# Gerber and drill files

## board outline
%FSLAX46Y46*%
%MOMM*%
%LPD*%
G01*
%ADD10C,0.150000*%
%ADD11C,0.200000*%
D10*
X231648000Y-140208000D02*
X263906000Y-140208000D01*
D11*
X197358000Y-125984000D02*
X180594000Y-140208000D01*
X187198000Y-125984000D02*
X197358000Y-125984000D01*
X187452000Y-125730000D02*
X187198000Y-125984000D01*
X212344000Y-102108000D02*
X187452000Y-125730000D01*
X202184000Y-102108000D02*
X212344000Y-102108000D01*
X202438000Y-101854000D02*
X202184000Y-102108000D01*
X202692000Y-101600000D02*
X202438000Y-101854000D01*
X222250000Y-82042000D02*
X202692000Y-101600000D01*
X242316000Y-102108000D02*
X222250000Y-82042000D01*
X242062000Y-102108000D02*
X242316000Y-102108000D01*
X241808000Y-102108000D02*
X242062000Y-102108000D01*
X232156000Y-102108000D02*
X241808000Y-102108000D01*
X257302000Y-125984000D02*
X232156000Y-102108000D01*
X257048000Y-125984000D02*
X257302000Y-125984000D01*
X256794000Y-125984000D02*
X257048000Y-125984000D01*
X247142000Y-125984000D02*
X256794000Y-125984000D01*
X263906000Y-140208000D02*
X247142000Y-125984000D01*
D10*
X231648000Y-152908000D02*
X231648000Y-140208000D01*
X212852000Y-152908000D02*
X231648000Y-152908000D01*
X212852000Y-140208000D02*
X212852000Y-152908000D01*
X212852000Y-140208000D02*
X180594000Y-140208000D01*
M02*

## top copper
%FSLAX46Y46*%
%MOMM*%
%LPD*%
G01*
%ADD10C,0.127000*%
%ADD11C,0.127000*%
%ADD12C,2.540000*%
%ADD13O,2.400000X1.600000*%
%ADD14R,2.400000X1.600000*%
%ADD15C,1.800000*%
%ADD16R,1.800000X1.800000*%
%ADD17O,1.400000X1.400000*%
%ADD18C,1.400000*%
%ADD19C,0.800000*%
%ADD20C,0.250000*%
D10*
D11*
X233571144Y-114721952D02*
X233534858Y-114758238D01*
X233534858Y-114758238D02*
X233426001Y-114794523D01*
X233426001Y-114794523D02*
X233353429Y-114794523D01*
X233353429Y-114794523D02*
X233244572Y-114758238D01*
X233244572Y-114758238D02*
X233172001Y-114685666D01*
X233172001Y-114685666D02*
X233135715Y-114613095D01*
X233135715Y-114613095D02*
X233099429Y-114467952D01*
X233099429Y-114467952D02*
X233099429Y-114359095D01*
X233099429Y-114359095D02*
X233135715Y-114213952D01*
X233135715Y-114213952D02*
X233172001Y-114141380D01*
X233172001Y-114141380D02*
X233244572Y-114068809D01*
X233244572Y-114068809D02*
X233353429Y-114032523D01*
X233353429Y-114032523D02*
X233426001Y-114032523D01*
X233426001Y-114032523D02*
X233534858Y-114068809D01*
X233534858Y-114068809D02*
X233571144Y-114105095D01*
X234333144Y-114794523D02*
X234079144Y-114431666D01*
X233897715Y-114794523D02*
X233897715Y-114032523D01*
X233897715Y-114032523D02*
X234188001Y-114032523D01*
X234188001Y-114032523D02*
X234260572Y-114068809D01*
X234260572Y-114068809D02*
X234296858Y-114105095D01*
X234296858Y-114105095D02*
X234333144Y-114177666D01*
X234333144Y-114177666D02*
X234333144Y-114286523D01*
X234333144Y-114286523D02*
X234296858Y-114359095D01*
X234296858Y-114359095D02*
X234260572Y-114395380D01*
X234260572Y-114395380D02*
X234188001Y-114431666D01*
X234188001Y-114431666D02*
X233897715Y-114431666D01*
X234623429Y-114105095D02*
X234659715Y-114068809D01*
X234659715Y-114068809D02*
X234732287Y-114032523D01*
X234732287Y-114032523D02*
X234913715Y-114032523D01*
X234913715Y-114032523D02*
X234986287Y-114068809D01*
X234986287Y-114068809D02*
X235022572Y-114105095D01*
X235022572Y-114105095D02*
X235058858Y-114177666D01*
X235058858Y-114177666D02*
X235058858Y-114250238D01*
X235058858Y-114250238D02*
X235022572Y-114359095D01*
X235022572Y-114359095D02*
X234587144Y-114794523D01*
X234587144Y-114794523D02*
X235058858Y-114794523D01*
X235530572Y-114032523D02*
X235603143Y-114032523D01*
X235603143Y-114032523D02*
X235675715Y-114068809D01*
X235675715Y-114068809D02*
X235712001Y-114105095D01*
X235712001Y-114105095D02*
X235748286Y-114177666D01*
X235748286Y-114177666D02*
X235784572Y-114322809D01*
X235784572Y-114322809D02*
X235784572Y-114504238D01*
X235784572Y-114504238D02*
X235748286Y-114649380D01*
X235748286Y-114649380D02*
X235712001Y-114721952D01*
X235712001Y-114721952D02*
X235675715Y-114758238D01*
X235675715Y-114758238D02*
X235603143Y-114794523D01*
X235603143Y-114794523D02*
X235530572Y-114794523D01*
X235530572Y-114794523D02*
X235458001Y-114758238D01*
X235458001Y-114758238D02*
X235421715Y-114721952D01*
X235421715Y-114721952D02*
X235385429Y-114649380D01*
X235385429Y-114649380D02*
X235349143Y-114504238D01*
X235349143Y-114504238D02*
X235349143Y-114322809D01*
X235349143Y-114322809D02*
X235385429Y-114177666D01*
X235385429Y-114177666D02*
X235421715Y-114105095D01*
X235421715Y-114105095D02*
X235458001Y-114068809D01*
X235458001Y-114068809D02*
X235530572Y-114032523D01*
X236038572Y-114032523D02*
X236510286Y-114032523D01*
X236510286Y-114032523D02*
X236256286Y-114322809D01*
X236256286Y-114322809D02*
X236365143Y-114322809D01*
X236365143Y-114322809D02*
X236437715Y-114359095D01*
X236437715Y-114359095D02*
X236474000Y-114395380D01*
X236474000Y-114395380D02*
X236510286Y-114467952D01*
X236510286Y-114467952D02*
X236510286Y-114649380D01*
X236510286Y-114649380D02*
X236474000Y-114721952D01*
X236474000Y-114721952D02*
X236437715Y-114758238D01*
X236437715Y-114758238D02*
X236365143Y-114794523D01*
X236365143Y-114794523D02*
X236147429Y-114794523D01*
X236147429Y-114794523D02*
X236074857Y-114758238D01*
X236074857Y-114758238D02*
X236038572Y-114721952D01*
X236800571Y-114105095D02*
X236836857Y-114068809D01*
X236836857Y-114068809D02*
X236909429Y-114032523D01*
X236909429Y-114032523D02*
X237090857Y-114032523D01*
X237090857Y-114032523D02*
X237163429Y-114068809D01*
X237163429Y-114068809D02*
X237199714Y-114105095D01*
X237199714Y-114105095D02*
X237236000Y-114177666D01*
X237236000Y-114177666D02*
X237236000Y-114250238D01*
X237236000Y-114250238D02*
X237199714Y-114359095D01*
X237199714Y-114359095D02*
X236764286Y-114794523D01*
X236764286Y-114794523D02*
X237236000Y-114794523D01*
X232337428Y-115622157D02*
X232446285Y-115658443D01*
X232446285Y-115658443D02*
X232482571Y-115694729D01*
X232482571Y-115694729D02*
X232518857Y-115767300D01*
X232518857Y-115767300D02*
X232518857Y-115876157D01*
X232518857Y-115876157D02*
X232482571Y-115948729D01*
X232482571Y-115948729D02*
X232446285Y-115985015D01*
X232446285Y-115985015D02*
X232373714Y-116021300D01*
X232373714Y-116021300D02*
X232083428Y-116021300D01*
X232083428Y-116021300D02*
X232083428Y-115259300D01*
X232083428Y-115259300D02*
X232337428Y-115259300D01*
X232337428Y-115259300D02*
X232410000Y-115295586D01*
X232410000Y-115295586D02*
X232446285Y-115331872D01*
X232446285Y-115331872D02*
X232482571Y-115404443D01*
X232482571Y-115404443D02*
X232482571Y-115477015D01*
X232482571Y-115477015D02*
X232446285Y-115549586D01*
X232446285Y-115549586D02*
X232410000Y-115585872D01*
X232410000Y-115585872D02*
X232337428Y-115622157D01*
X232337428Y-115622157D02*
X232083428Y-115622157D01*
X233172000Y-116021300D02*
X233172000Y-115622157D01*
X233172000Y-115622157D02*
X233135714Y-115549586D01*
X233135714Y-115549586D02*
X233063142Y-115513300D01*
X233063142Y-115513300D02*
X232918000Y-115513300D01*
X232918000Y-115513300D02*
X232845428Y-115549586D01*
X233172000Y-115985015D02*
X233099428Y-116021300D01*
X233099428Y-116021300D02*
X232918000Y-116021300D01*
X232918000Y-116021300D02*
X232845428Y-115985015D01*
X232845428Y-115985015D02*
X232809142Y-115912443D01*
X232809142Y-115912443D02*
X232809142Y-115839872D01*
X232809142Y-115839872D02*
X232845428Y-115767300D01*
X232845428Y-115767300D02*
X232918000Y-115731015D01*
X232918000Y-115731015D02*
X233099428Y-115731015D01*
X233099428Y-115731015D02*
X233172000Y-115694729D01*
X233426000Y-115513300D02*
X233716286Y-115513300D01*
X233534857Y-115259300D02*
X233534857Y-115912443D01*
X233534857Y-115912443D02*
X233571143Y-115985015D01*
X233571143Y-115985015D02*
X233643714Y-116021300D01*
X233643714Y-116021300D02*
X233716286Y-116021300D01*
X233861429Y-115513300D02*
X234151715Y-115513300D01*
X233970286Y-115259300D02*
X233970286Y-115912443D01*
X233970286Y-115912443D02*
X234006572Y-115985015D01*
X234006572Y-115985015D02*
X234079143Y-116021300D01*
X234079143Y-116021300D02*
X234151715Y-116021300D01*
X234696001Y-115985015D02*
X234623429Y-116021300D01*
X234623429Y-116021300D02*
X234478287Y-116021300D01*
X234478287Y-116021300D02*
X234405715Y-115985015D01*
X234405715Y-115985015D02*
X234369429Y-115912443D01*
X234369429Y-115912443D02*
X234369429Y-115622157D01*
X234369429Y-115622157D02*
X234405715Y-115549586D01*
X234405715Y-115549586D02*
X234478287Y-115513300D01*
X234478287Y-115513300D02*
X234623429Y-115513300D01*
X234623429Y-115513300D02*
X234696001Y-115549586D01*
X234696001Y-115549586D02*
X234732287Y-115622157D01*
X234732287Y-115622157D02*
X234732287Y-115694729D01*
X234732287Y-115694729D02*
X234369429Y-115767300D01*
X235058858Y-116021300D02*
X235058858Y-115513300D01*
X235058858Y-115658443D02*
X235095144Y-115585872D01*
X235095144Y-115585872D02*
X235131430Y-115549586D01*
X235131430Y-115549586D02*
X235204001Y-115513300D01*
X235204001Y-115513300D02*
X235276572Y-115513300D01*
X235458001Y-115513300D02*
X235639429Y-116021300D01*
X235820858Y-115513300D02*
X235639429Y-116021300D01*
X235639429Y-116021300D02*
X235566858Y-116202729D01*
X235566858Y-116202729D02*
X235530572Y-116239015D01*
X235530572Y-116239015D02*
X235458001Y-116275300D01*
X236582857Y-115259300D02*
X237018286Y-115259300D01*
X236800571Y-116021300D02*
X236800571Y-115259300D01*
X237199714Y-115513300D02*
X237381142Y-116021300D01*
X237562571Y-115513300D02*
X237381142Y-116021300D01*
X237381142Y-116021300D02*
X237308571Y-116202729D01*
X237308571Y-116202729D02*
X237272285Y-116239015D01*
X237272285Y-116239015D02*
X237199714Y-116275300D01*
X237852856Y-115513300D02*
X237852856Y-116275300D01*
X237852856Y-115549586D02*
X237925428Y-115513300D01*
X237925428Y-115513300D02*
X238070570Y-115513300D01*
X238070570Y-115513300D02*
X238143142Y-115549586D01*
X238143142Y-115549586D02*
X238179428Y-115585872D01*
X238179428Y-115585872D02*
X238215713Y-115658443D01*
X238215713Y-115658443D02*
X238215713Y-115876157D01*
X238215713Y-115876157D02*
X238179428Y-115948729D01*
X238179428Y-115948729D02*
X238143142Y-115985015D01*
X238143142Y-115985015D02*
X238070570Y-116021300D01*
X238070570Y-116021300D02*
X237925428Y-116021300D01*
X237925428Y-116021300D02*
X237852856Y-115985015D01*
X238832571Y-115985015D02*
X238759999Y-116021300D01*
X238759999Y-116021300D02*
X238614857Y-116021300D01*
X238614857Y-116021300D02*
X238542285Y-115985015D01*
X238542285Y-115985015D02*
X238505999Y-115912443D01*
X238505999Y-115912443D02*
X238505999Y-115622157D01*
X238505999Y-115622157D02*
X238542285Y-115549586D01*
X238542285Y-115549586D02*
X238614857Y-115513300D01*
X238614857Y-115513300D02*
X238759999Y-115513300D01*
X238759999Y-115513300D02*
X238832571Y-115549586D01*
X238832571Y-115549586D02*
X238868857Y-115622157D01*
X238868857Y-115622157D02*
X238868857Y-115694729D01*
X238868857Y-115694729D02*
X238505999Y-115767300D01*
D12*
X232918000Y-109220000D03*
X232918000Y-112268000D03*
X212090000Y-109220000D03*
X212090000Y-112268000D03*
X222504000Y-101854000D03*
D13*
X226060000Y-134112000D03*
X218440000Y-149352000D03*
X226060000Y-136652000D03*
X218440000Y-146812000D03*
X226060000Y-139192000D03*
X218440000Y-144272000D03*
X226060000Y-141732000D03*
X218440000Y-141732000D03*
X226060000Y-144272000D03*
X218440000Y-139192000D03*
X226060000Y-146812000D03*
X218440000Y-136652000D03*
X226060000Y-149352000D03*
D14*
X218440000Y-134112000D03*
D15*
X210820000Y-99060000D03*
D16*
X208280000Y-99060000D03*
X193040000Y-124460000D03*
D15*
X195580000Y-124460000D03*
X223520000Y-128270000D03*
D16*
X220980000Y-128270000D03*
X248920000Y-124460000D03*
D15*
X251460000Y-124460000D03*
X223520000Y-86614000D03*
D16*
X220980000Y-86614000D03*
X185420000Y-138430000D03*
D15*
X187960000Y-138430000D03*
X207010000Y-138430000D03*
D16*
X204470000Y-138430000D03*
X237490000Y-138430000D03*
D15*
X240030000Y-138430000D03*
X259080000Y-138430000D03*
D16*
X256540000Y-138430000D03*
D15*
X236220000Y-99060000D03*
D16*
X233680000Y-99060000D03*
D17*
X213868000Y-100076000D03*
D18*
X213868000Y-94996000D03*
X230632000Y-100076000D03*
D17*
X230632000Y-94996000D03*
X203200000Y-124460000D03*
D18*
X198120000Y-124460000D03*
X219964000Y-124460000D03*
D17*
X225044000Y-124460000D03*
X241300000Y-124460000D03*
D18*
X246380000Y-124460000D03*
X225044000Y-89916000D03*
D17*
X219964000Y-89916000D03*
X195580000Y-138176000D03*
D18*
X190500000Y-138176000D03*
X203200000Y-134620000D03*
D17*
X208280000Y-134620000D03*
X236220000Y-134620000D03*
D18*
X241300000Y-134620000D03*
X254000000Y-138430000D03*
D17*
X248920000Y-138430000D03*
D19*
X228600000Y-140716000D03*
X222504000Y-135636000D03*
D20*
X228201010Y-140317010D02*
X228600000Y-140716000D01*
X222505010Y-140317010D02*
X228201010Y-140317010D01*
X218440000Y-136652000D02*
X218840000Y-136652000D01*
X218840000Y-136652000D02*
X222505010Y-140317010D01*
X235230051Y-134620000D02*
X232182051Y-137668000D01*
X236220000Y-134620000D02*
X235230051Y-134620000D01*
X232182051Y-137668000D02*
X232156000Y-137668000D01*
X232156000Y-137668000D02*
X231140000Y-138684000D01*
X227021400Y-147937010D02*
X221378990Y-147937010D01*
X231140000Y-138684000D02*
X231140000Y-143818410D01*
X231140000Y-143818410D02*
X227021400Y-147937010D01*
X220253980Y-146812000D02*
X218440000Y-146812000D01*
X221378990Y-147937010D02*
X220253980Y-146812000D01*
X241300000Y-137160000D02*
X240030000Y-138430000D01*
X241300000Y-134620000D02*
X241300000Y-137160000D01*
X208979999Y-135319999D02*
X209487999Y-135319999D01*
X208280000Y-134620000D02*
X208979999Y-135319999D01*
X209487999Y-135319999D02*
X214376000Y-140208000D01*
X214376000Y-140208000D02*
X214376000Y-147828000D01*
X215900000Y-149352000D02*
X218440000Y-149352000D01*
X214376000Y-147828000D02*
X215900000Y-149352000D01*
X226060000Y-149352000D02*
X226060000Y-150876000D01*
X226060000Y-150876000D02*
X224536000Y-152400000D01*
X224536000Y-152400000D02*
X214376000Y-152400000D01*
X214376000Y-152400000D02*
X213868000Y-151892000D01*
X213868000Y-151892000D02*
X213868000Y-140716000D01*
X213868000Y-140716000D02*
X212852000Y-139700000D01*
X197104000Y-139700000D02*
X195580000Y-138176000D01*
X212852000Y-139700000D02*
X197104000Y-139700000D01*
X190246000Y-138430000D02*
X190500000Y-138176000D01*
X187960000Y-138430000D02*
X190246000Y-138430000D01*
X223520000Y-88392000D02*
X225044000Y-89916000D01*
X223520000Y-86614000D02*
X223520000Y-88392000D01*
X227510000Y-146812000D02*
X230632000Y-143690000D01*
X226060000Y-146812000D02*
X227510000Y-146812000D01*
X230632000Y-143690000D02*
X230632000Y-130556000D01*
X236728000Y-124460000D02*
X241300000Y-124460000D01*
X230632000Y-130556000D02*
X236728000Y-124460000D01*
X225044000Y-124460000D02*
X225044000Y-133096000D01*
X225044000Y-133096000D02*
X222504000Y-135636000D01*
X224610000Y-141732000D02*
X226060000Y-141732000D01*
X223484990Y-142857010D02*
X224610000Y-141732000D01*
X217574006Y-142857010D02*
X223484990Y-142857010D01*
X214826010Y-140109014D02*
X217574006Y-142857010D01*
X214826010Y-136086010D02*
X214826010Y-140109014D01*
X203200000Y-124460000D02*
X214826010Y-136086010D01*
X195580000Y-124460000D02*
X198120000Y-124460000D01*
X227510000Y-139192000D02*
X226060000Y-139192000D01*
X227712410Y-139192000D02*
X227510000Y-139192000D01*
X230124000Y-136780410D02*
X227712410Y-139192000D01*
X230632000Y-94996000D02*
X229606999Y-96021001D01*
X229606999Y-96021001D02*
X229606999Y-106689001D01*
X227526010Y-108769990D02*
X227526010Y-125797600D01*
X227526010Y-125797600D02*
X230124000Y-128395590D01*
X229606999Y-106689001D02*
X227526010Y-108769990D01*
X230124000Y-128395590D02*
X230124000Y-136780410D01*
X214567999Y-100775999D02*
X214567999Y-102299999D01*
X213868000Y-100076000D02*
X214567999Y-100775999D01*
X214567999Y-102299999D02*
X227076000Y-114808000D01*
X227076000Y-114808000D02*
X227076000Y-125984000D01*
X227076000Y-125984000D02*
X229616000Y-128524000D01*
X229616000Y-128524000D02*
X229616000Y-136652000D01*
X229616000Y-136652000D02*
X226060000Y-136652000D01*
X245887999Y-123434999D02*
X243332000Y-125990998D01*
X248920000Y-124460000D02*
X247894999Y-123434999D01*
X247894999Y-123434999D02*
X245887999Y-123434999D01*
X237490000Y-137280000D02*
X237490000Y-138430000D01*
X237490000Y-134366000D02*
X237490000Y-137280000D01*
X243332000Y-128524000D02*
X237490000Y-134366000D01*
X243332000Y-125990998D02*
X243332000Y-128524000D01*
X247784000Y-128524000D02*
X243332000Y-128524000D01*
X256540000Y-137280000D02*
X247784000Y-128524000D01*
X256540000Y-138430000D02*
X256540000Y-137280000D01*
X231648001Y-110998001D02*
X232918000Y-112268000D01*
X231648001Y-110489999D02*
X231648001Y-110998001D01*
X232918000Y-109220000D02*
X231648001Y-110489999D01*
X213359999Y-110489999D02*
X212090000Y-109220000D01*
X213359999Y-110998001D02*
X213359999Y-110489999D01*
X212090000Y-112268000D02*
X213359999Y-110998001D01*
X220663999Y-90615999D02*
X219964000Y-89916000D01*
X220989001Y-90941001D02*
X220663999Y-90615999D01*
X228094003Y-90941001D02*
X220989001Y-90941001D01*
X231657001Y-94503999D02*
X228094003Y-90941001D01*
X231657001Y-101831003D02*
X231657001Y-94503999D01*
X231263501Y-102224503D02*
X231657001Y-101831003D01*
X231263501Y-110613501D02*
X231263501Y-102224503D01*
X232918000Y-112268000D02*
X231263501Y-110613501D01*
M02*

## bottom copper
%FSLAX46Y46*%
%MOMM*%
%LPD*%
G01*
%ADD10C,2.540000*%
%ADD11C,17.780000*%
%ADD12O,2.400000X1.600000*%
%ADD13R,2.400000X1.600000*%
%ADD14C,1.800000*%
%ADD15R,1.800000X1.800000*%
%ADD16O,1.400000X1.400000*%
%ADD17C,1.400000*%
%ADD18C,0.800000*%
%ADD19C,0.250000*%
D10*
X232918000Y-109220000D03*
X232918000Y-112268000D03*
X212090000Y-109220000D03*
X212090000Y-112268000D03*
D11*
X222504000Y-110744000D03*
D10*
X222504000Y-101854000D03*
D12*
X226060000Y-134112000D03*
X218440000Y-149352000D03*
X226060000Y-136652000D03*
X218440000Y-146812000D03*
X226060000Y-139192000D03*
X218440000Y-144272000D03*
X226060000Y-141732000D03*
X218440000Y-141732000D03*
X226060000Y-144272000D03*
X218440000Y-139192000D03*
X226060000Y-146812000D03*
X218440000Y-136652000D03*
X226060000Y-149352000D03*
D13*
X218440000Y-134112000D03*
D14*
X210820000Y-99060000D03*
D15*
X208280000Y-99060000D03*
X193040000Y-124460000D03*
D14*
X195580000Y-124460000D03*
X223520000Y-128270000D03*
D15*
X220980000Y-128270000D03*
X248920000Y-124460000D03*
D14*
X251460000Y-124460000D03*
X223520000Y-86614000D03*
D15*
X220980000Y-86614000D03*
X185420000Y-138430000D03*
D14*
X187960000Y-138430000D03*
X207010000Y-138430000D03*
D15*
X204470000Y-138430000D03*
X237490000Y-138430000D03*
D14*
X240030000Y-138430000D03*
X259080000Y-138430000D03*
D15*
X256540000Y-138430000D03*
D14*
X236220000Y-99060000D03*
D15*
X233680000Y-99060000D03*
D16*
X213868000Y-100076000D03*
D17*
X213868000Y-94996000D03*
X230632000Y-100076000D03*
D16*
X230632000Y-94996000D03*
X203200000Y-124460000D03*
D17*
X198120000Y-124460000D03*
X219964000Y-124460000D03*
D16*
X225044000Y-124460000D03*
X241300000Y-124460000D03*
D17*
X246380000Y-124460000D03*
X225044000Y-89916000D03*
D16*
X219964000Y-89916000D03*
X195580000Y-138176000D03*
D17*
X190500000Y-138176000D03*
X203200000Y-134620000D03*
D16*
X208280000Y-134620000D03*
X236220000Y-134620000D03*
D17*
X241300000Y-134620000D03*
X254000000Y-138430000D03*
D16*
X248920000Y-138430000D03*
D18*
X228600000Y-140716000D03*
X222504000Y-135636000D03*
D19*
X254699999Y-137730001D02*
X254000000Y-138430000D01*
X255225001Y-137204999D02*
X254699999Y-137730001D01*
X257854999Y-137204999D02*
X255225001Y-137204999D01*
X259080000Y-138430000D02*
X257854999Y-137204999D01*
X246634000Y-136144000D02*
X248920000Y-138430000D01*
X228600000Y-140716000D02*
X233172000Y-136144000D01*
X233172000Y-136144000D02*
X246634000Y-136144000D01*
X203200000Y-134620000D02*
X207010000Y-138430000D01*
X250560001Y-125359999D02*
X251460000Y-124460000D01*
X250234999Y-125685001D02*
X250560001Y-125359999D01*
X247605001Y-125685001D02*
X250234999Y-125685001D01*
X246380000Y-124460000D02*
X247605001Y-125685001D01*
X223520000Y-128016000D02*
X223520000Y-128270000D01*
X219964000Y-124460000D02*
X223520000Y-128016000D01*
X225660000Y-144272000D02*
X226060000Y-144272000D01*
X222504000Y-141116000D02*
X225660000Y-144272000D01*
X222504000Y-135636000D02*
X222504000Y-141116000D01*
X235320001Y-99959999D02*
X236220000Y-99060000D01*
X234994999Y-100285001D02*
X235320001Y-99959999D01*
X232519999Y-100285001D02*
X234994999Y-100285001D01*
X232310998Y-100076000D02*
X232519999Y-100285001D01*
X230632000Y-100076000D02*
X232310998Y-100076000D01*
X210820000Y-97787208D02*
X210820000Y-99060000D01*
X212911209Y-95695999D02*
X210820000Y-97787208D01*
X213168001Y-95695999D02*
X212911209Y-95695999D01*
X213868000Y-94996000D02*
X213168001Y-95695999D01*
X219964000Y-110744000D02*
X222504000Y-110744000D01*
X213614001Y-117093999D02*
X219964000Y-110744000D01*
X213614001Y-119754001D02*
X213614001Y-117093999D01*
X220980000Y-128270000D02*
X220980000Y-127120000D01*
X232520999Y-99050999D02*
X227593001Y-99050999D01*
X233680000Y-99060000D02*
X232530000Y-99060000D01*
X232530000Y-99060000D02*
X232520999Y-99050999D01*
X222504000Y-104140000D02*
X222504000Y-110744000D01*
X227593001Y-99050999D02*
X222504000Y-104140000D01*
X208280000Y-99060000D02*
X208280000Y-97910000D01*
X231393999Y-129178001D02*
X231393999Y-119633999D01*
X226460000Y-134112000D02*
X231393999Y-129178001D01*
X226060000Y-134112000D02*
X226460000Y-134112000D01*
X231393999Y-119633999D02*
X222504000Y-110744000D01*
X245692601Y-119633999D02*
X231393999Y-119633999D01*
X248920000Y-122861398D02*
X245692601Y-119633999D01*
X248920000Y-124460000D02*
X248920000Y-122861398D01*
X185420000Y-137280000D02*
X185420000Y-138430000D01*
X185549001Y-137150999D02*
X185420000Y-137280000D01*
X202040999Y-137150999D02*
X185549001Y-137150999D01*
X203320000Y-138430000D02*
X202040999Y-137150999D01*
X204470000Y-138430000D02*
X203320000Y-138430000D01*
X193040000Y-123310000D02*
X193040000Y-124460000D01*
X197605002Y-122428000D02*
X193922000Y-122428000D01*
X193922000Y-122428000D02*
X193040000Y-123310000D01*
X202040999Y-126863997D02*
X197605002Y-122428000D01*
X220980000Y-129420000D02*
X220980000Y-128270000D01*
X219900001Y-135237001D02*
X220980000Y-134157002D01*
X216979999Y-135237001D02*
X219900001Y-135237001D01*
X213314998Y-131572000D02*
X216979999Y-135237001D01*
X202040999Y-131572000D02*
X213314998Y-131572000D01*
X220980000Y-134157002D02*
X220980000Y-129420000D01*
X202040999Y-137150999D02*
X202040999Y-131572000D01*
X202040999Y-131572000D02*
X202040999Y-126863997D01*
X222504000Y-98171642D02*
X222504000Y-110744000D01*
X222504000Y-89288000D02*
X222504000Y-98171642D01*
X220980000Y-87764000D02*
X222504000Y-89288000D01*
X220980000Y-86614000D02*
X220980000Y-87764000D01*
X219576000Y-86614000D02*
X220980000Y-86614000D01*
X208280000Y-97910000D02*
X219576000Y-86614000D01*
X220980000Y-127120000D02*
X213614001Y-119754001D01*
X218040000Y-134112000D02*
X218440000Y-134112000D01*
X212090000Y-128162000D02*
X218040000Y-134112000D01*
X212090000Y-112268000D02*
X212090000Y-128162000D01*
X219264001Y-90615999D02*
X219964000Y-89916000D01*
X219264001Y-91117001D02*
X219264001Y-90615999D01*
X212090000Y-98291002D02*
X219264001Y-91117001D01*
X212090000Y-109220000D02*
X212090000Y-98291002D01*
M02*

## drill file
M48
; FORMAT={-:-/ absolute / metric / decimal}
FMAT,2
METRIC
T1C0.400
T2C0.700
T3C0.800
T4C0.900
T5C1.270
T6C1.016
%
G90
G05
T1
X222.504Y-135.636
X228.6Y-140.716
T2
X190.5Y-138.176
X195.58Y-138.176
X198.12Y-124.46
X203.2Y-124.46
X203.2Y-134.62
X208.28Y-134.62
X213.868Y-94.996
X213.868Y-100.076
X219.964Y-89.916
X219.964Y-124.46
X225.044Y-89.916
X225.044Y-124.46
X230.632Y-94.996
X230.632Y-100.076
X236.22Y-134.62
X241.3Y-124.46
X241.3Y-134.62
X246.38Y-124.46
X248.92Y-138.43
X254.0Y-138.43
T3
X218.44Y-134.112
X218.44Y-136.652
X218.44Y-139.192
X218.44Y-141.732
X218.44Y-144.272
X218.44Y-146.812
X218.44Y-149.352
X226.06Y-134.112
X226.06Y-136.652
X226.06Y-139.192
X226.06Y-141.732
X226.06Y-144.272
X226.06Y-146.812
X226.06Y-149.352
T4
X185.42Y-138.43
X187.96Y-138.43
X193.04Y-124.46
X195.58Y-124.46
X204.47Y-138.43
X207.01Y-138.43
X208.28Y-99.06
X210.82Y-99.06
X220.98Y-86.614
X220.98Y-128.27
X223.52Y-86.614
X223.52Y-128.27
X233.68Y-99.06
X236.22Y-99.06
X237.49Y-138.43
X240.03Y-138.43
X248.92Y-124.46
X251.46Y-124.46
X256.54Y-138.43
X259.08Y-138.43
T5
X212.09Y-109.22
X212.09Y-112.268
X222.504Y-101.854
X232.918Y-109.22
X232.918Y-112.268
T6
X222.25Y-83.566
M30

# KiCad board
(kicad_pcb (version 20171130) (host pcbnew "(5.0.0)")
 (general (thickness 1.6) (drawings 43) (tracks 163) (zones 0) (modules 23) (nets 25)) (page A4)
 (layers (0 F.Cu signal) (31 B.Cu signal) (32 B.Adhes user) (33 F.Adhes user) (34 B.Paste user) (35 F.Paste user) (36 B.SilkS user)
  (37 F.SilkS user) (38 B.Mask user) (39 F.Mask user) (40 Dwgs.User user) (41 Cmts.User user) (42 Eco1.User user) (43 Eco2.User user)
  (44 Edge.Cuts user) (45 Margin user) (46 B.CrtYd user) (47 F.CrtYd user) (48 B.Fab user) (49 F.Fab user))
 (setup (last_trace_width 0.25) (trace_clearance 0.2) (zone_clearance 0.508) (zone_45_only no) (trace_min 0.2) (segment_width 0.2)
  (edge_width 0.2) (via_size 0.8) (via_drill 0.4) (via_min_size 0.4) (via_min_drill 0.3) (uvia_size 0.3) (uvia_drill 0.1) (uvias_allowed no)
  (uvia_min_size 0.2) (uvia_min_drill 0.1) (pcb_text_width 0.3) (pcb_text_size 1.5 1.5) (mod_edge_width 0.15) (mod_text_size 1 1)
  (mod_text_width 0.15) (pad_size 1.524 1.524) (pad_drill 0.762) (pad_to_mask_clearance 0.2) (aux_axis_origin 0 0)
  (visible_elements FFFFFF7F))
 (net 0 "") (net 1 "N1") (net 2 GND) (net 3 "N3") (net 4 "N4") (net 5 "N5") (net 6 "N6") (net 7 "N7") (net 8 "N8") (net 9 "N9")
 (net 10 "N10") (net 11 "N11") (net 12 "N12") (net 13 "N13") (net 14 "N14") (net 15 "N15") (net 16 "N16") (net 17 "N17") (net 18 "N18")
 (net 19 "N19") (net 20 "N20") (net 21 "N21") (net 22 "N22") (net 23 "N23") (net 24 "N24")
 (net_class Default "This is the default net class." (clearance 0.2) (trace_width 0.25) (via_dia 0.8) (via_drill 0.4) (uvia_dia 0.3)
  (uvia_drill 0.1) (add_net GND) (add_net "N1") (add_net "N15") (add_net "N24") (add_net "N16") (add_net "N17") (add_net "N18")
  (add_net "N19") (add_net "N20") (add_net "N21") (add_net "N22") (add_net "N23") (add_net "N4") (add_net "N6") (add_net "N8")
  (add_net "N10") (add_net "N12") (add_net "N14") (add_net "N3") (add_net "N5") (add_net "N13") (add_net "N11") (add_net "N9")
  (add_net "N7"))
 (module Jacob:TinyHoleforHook (layer F.Cu) (at 222.25 83.566)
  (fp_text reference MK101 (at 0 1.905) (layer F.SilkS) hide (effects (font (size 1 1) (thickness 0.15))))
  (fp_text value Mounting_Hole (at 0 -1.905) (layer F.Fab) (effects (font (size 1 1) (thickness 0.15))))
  (pad "" np_thru_hole circle (at 0 0) (size 1.016 1.016) (drill 1.016) (layers *.Cu *.Mask)))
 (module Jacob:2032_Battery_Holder (layer B.Cu) (at 222.504 110.744)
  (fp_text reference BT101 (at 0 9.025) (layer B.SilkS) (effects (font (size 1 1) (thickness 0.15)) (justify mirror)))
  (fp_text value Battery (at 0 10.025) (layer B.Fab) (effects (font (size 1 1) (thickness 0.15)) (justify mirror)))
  (pad 1 thru_hole circle (at 10.414 -1.524) (size 2.54 2.54) (drill 1.27) (layers *.Cu *.Mask) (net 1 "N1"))
  (pad 1 thru_hole circle (at 10.414 1.524) (size 2.54 2.54) (drill 1.27) (layers *.Cu *.Mask) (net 1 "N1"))
  (pad 1 thru_hole circle (at -10.414 -1.524) (size 2.54 2.54) (drill 1.27) (layers *.Cu *.Mask) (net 1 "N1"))
  (pad 1 thru_hole circle (at -10.414 1.524) (size 2.54 2.54) (drill 1.27) (layers *.Cu *.Mask) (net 1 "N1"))
  (pad 2 smd circle (at 0 0) (size 17.78 17.78) (layers B.Cu B.Paste B.Mask) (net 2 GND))
  (pad 2 thru_hole circle (at 0 -8.89) (size 2.54 2.54) (drill 1.27) (layers *.Cu *.Mask) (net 2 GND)))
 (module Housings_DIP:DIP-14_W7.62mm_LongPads (layer F.Cu) (at 218.44 134.112)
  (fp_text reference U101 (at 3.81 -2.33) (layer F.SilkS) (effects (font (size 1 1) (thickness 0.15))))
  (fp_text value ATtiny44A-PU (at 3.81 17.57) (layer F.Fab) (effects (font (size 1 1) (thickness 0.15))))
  (pad 14 thru_hole oval (at 7.62 0) (size 2.4 1.6) (drill 0.8) (layers *.Cu *.Mask) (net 2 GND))
  (pad 7 thru_hole oval (at 0 15.24) (size 2.4 1.6) (drill 0.8) (layers *.Cu *.Mask) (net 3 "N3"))
  (pad 13 thru_hole oval (at 7.62 2.54) (size 2.4 1.6) (drill 0.8) (layers *.Cu *.Mask) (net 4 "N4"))
  (pad 6 thru_hole oval (at 0 12.7) (size 2.4 1.6) (drill 0.8) (layers *.Cu *.Mask) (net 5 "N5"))
  (pad 12 thru_hole oval (at 7.62 5.08) (size 2.4 1.6) (drill 0.8) (layers *.Cu *.Mask) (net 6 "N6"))
  (pad 5 thru_hole oval (at 0 10.16) (size 2.4 1.6) (drill 0.8) (layers *.Cu *.Mask) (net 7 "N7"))
  (pad 11 thru_hole oval (at 7.62 7.62) (size 2.4 1.6) (drill 0.8) (layers *.Cu *.Mask) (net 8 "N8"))
  (pad 4 thru_hole oval (at 0 7.62) (size 2.4 1.6) (drill 0.8) (layers *.Cu *.Mask) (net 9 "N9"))
  (pad 10 thru_hole oval (at 7.62 10.16) (size 2.4 1.6) (drill 0.8) (layers *.Cu *.Mask) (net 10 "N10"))
  (pad 3 thru_hole oval (at 0 5.08) (size 2.4 1.6) (drill 0.8) (layers *.Cu *.Mask) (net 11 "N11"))
  (pad 9 thru_hole oval (at 7.62 12.7) (size 2.4 1.6) (drill 0.8) (layers *.Cu *.Mask) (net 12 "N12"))
  (pad 2 thru_hole oval (at 0 2.54) (size 2.4 1.6) (drill 0.8) (layers *.Cu *.Mask) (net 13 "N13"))
  (pad 8 thru_hole oval (at 7.62 15.24) (size 2.4 1.6) (drill 0.8) (layers *.Cu *.Mask) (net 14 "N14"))
  (pad 1 thru_hole rect (at 0 0) (size 2.4 1.6) (drill 0.8) (layers *.Cu *.Mask) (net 1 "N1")))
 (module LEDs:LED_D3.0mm (layer F.Cu) (at 208.28 99.06)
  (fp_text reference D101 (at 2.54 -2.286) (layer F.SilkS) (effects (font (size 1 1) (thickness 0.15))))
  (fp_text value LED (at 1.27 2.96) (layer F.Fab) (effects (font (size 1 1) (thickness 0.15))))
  (pad 2 thru_hole circle (at 2.54 0) (size 1.8 1.8) (drill 0.9) (layers *.Cu *.Mask) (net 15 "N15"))
  (pad 1 thru_hole rect (at 0 0) (size 1.8 1.8) (drill 0.9) (layers *.Cu *.Mask) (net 2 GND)))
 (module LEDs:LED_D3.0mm (layer F.Cu) (at 193.04 124.46)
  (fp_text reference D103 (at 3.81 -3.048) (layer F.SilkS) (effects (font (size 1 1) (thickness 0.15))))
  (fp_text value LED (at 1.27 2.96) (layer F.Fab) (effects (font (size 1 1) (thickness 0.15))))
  (pad 1 thru_hole rect (at 0 0) (size 1.8 1.8) (drill 0.9) (layers *.Cu *.Mask) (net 2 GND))
  (pad 2 thru_hole circle (at 2.54 0) (size 1.8 1.8) (drill 0.9) (layers *.Cu *.Mask) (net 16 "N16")))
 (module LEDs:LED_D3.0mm (layer F.Cu) (at 220.98 128.27)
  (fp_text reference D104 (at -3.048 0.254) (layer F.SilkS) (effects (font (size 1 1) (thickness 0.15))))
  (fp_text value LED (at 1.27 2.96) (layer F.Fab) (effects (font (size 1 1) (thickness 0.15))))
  (pad 2 thru_hole circle (at 2.54 0) (size 1.8 1.8) (drill 0.9) (layers *.Cu *.Mask) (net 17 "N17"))
  (pad 1 thru_hole rect (at 0 0) (size 1.8 1.8) (drill 0.9) (layers *.Cu *.Mask) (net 2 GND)))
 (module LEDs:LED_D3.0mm (layer F.Cu) (at 248.92 124.46)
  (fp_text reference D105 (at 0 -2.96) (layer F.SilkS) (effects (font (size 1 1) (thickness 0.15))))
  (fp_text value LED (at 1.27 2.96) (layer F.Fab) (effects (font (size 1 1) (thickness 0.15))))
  (pad 1 thru_hole rect (at 0 0) (size 1.8 1.8) (drill 0.9) (layers *.Cu *.Mask) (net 2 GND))
  (pad 2 thru_hole circle (at 2.54 0) (size 1.8 1.8) (drill 0.9) (layers *.Cu *.Mask) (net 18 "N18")))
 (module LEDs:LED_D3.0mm (layer F.Cu) (at 220.98 86.614)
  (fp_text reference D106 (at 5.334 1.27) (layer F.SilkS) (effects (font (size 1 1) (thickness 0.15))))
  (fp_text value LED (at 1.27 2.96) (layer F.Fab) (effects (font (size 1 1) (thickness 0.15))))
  (pad 2 thru_hole circle (at 2.54 0) (size 1.8 1.8) (drill 0.9) (layers *.Cu *.Mask) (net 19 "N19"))
  (pad 1 thru_hole rect (at 0 0) (size 1.8 1.8) (drill 0.9) (layers *.Cu *.Mask) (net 2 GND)))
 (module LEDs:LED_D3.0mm (layer F.Cu) (at 185.42 138.43)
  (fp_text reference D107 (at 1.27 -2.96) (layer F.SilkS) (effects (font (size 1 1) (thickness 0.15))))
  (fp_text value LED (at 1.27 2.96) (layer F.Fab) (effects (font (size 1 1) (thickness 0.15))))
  (pad 1 thru_hole rect (at 0 0) (size 1.8 1.8) (drill 0.9) (layers *.Cu *.Mask) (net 2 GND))
  (pad 2 thru_hole circle (at 2.54 0) (size 1.8 1.8) (drill 0.9) (layers *.Cu *.Mask) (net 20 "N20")))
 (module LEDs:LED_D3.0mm (layer F.Cu) (at 204.47 138.43)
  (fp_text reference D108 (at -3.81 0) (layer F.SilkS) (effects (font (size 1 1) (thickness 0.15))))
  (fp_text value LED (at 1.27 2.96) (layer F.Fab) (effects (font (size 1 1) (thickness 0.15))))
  (pad 2 thru_hole circle (at 2.54 0) (size 1.8 1.8) (drill 0.9) (layers *.Cu *.Mask) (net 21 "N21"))
  (pad 1 thru_hole rect (at 0 0) (size 1.8 1.8) (drill 0.9) (layers *.Cu *.Mask) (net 2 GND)))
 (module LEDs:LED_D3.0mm (layer F.Cu) (at 237.49 138.43)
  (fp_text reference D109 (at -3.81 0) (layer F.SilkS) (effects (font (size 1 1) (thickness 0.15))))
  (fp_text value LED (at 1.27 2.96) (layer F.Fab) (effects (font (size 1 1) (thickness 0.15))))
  (pad 1 thru_hole rect (at 0 0) (size 1.8 1.8) (drill 0.9) (layers *.Cu *.Mask) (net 2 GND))
  (pad 2 thru_hole circle (at 2.54 0) (size 1.8 1.8) (drill 0.9) (layers *.Cu *.Mask) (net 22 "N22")))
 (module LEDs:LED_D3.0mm (layer F.Cu) (at 256.54 138.43)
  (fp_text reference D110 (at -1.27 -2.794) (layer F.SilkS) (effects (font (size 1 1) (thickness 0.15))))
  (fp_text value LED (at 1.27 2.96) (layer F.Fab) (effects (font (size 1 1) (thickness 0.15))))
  (pad 2 thru_hole circle (at 2.54 0) (size 1.8 1.8) (drill 0.9) (layers *.Cu *.Mask) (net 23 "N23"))
  (pad 1 thru_hole rect (at 0 0) (size 1.8 1.8) (drill 0.9) (layers *.Cu *.Mask) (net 2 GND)))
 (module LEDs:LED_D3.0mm (layer F.Cu) (at 233.68 99.06)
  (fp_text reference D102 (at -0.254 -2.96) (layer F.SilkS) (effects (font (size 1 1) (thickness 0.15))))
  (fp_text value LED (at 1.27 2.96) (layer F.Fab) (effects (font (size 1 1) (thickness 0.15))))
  (pad 2 thru_hole circle (at 2.54 0) (size 1.8 1.8) (drill 0.9) (layers *.Cu *.Mask) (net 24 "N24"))
  (pad 1 thru_hole rect (at 0 0) (size 1.8 1.8) (drill 0.9) (layers *.Cu *.Mask) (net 2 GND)))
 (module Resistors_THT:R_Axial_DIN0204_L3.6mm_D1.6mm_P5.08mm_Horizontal (layer F.Cu) (at 213.868 94.996 270)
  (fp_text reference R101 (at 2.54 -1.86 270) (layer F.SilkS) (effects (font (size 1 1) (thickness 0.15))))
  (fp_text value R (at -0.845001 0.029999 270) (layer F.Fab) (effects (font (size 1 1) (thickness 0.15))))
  (pad 2 thru_hole oval (at 5.08 0 270) (size 1.4 1.4) (drill 0.7) (layers *.Cu *.Mask) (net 4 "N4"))
  (pad 1 thru_hole circle (at 0 0 270) (size 1.4 1.4) (drill 0.7) (layers *.Cu *.Mask) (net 15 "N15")))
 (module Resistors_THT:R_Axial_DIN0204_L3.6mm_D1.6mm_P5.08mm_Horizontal (layer F.Cu) (at 230.632 100.076 90)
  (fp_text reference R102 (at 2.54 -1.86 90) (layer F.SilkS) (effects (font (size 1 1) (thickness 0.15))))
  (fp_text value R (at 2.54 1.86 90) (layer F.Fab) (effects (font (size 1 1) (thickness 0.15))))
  (pad 1 thru_hole circle (at 0 0 90) (size 1.4 1.4) (drill 0.7) (layers *.Cu *.Mask) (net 24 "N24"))
  (pad 2 thru_hole oval (at 5.08 0 90) (size 1.4 1.4) (drill 0.7) (layers *.Cu *.Mask) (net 6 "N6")))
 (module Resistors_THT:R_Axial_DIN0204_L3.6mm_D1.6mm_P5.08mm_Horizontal (layer F.Cu) (at 198.12 124.46)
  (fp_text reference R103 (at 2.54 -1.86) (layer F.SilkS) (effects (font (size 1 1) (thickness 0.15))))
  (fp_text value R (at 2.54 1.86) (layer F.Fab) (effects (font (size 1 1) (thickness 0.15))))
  (pad 2 thru_hole oval (at 5.08 0) (size 1.4 1.4) (drill 0.7) (layers *.Cu *.Mask) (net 8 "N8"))
  (pad 1 thru_hole circle (at 0 0) (size 1.4 1.4) (drill 0.7) (layers *.Cu *.Mask) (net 16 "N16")))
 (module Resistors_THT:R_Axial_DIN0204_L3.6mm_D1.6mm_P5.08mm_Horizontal (layer F.Cu) (at 219.964 124.46)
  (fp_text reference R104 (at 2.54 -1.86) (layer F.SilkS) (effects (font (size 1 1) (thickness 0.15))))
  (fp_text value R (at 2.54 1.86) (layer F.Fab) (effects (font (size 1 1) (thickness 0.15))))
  (pad 1 thru_hole circle (at 0 0) (size 1.4 1.4) (drill 0.7) (layers *.Cu *.Mask) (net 17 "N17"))
  (pad 2 thru_hole oval (at 5.08 0) (size 1.4 1.4) (drill 0.7) (layers *.Cu *.Mask) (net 10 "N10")))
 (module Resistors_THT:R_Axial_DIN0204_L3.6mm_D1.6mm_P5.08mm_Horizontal (layer F.Cu) (at 246.38 124.46 180)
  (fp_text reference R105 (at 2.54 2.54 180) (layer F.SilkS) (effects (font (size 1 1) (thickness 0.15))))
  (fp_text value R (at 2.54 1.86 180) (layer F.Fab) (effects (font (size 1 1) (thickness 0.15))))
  (pad 2 thru_hole oval (at 5.08 0 180) (size 1.4 1.4) (drill 0.7) (layers *.Cu *.Mask) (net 12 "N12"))
  (pad 1 thru_hole circle (at 0 0 180) (size 1.4 1.4) (drill 0.7) (layers *.Cu *.Mask) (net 18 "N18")))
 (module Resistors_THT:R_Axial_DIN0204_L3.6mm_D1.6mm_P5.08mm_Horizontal (layer F.Cu) (at 225.044 89.916 180)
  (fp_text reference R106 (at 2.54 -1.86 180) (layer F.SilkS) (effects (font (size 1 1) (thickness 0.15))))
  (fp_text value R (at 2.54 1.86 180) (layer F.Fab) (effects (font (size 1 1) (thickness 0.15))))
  (pad 1 thru_hole circle (at 0 0 180) (size 1.4 1.4) (drill 0.7) (layers *.Cu *.Mask) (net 19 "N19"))
  (pad 2 thru_hole oval (at 5.08 0 180) (size 1.4 1.4) (drill 0.7) (layers *.Cu *.Mask) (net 1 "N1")))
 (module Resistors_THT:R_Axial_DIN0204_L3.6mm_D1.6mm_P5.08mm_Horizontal (layer F.Cu) (at 190.5 138.176)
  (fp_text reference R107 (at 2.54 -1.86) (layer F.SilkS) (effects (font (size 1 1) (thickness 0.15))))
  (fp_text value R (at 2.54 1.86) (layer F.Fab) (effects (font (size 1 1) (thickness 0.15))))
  (pad 2 thru_hole oval (at 5.08 0) (size 1.4 1.4) (drill 0.7) (layers *.Cu *.Mask) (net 14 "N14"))
  (pad 1 thru_hole circle (at 0 0) (size 1.4 1.4) (drill 0.7) (layers *.Cu *.Mask) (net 20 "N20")))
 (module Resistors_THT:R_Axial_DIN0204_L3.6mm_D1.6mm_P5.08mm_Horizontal (layer F.Cu) (at 203.2 134.62)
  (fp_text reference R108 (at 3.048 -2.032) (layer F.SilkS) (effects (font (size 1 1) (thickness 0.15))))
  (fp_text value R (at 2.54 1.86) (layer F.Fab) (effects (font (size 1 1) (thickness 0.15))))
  (pad 1 thru_hole circle (at 0 0) (size 1.4 1.4) (drill 0.7) (layers *.Cu *.Mask) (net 21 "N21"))
  (pad 2 thru_hole oval (at 5.08 0) (size 1.4 1.4) (drill 0.7) (layers *.Cu *.Mask) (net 3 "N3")))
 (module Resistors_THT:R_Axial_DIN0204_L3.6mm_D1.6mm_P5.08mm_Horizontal (layer F.Cu) (at 241.3 134.62 180)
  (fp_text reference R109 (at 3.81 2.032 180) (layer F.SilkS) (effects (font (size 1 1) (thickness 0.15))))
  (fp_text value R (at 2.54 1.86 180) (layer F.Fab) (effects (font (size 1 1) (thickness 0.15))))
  (pad 2 thru_hole oval (at 5.08 0 180) (size 1.4 1.4) (drill 0.7) (layers *.Cu *.Mask) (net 5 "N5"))
  (pad 1 thru_hole circle (at 0 0 180) (size 1.4 1.4) (drill 0.7) (layers *.Cu *.Mask) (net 22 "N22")))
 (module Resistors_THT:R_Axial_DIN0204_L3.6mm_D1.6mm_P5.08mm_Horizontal (layer F.Cu) (at 254 138.43 180)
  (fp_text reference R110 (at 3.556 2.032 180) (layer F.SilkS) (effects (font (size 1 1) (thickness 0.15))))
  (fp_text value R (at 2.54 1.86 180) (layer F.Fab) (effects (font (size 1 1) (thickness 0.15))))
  (pad 1 thru_hole circle (at 0 0 180) (size 1.4 1.4) (drill 0.7) (layers *.Cu *.Mask) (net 23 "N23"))
  (pad 2 thru_hole oval (at 5.08 0 180) (size 1.4 1.4) (drill 0.7) (layers *.Cu *.Mask) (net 13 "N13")))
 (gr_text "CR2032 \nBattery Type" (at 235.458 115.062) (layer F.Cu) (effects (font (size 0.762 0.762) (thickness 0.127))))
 (gr_line (start 231.648 140.208) (end 263.906 140.208) (layer Edge.Cuts) (width 0.15))
 (gr_line (start 197.358 125.984) (end 180.594 140.208) (layer Edge.Cuts) (width 0.2))
 (gr_line (start 187.198 125.984) (end 197.358 125.984) (layer Edge.Cuts) (width 0.2))
 (gr_line (start 187.452 125.73) (end 187.198 125.984) (layer Edge.Cuts) (width 0.2))
 (gr_line (start 212.344 102.108) (end 187.452 125.73) (layer Edge.Cuts) (width 0.2))
 (gr_line (start 202.184 102.108) (end 212.344 102.108) (layer Edge.Cuts) (width 0.2))
 (gr_line (start 202.438 101.854) (end 202.184 102.108) (layer Edge.Cuts) (width 0.2))
 (gr_line (start 202.692 101.6) (end 202.438 101.854) (layer Edge.Cuts) (width 0.2))
 (gr_line (start 222.25 82.042) (end 202.692 101.6) (layer Edge.Cuts) (width 0.2))
 (gr_line (start 242.316 102.108) (end 222.25 82.042) (layer Edge.Cuts) (width 0.2))
 (gr_line (start 242.062 102.108) (end 242.316 102.108) (layer Edge.Cuts) (width 0.2))
 (gr_line (start 241.808 102.108) (end 242.062 102.108) (layer Edge.Cuts) (width 0.2))
 (gr_line (start 232.156 102.108) (end 241.808 102.108) (layer Edge.Cuts) (width 0.2))
 (gr_line (start 257.302 125.984) (end 232.156 102.108) (layer Edge.Cuts) (width 0.2))
 (gr_line (start 257.048 125.984) (end 257.302 125.984) (layer Edge.Cuts) (width 0.2))
 (gr_line (start 256.794 125.984) (end 257.048 125.984) (layer Edge.Cuts) (width 0.2))
 (gr_line (start 247.142 125.984) (end 256.794 125.984) (layer Edge.Cuts) (width 0.2))
 (gr_line (start 263.906 140.208) (end 247.142 125.984) (layer Edge.Cuts) (width 0.2))
 (gr_line (start 231.648 152.908) (end 231.648 140.208) (layer Edge.Cuts) (width 0.15))
 (gr_line (start 212.852 152.908) (end 231.648 152.908) (layer Edge.Cuts) (width 0.15))
 (gr_line (start 212.852 140.208) (end 212.852 152.908) (layer Edge.Cuts) (width 0.15))
 (gr_line (start 212.852 140.208) (end 180.594 140.208) (layer Edge.Cuts) (width 0.15))
 (segment (start 254.699999 137.730001) (end 254 138.43) (width 0.25) (layer B.Cu) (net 23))
 (segment (start 255.225001 137.204999) (end 254.699999 137.730001) (width 0.25) (layer B.Cu) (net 23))
 (segment (start 257.854999 137.204999) (end 255.225001 137.204999) (width 0.25) (layer B.Cu) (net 23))
 (segment (start 259.08 138.43) (end 257.854999 137.204999) (width 0.25) (layer B.Cu) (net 23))
 (via (at 228.6 140.716) (size 0.8) (drill 0.4) (layers F.Cu B.Cu) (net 13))
 (segment (start 228.20101 140.31701) (end 228.6 140.716) (width 0.25) (layer F.Cu) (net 13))
 (segment (start 222.50501 140.31701) (end 228.20101 140.31701) (width 0.25) (layer F.Cu) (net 13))
 (segment (start 218.44 136.652) (end 218.84 136.652) (width 0.25) (layer F.Cu) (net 13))
 (segment (start 218.84 136.652) (end 222.50501 140.31701) (width 0.25) (layer F.Cu) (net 13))
 (segment (start 246.634 136.144) (end 248.92 138.43) (width 0.25) (layer B.Cu) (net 13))
 (segment (start 228.6 140.716) (end 233.172 136.144) (width 0.25) (layer B.Cu) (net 13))
 (segment (start 233.172 136.144) (end 246.634 136.144) (width 0.25) (layer B.Cu) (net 13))
 (segment (start 235.230051 134.62) (end 232.182051 137.668) (width 0.25) (layer F.Cu) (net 5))
 (segment (start 236.22 134.62) (end 235.230051 134.62) (width 0.25) (layer F.Cu) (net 5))
 (segment (start 232.182051 137.668) (end 232.156 137.668) (width 0.25) (layer F.Cu) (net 5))
 (segment (start 232.156 137.668) (end 231.14 138.684) (width 0.25) (layer F.Cu) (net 5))
 (segment (start 227.0214 147.93701) (end 221.37899 147.93701) (width 0.25) (layer F.Cu) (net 5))
 (segment (start 231.14 138.684) (end 231.14 143.81841) (width 0.25) (layer F.Cu) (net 5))
 (segment (start 231.14 143.81841) (end 227.0214 147.93701) (width 0.25) (layer F.Cu) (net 5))
 (segment (start 220.25398 146.812) (end 218.44 146.812) (width 0.25) (layer F.Cu) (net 5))
 (segment (start 221.37899 147.93701) (end 220.25398 146.812) (width 0.25) (layer F.Cu) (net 5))
 (segment (start 241.3 137.16) (end 240.03 138.43) (width 0.25) (layer F.Cu) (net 22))
 (segment (start 241.3 134.62) (end 241.3 137.16) (width 0.25) (layer F.Cu) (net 22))
 (segment (start 203.2 134.62) (end 207.01 138.43) (width 0.25) (layer B.Cu) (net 21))
 (segment (start 208.979999 135.319999) (end 209.487999 135.319999) (width 0.25) (layer F.Cu) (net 3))
 (segment (start 208.28 134.62) (end 208.979999 135.319999) (width 0.25) (layer F.Cu) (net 3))
 (segment (start 209.487999 135.319999) (end 214.376 140.208) (width 0.25) (layer F.Cu) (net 3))
 (segment (start 214.376 140.208) (end 214.376 147.828) (width 0.25) (layer F.Cu) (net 3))
 (segment (start 215.9 149.352) (end 218.44 149.352) (width 0.25) (layer F.Cu) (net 3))
 (segment (start 214.376 147.828) (end 215.9 149.352) (width 0.25) (layer F.Cu) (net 3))
 (segment (start 226.06 149.352) (end 226.06 150.876) (width 0.25) (layer F.Cu) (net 14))
 (segment (start 226.06 150.876) (end 224.536 152.4) (width 0.25) (layer F.Cu) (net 14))
 (segment (start 224.536 152.4) (end 214.376 152.4) (width 0.25) (layer F.Cu) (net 14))
 (segment (start 214.376 152.4) (end 213.868 151.892) (width 0.25) (layer F.Cu) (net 14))
 (segment (start 213.868 151.892) (end 213.868 140.716) (width 0.25) (layer F.Cu) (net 14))
 (segment (start 213.868 140.716) (end 212.852 139.7) (width 0.25) (layer F.Cu) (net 14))
 (segment (start 197.104 139.7) (end 195.58 138.176) (width 0.25) (layer F.Cu) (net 14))
 (segment (start 212.852 139.7) (end 197.104 139.7) (width 0.25) (layer F.Cu) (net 14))
 (segment (start 190.246 138.43) (end 190.5 138.176) (width 0.25) (layer F.Cu) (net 20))
 (segment (start 187.96 138.43) (end 190.246 138.43) (width 0.25) (layer F.Cu) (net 20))
 (segment (start 223.52 88.392) (end 225.044 89.916) (width 0.25) (layer F.Cu) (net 19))
 (segment (start 223.52 86.614) (end 223.52 88.392) (width 0.25) (layer F.Cu) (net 19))
 (segment (start 227.51 146.812) (end 230.632 143.69) (width 0.25) (layer F.Cu) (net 12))
 (segment (start 226.06 146.812) (end 227.51 146.812) (width 0.25) (layer F.Cu) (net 12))
 (segment (start 230.632 143.69) (end 230.632 130.556) (width 0.25) (layer F.Cu) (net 12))
 (segment (start 236.728 124.46) (end 241.3 124.46) (width 0.25) (layer F.Cu) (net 12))
 (segment (start 230.632 130.556) (end 236.728 124.46) (width 0.25) (layer F.Cu) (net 12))
 (segment (start 250.560001 125.359999) (end 251.46 124.46) (width 0.25) (layer B.Cu) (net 18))
 (segment (start 250.234999 125.685001) (end 250.560001 125.359999) (width 0.25) (layer B.Cu) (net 18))
 (segment (start 247.605001 125.685001) (end 250.234999 125.685001) (width 0.25) (layer B.Cu) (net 18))
 (segment (start 246.38 124.46) (end 247.605001 125.685001) (width 0.25) (layer B.Cu) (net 18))
 (segment (start 223.52 128.016) (end 223.52 128.27) (width 0.25) (layer B.Cu) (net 17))
 (segment (start 219.964 124.46) (end 223.52 128.016) (width 0.25) (layer B.Cu) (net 17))
 (via (at 222.504 135.636) (size 0.8) (drill 0.4) (layers F.Cu B.Cu) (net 10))
 (segment (start 225.044 124.46) (end 225.044 133.096) (width 0.25) (layer F.Cu) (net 10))
 (segment (start 225.044 133.096) (end 222.504 135.636) (width 0.25) (layer F.Cu) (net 10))
 (segment (start 225.66 144.272) (end 226.06 144.272) (width 0.25) (layer B.Cu) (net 10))
 (segment (start 222.504 141.116) (end 225.66 144.272) (width 0.25) (layer B.Cu) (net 10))
 (segment (start 222.504 135.636) (end 222.504 141.116) (width 0.25) (layer B.Cu) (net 10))
 (segment (start 224.61 141.732) (end 226.06 141.732) (width 0.25) (layer F.Cu) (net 8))
 (segment (start 223.48499 142.85701) (end 224.61 141.732) (width 0.25) (layer F.Cu) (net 8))
 (segment (start 217.574006 142.85701) (end 223.48499 142.85701) (width 0.25) (layer F.Cu) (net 8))
 (segment (start 214.82601 140.109014) (end 217.574006 142.85701) (width 0.25) (layer F.Cu) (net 8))
 (segment (start 214.82601 136.08601) (end 214.82601 140.109014) (width 0.25) (layer F.Cu) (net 8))
 (segment (start 203.2 124.46) (end 214.82601 136.08601) (width 0.25) (layer F.Cu) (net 8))
 (segment (start 195.58 124.46) (end 198.12 124.46) (width 0.25) (layer F.Cu) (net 16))
 (segment (start 235.320001 99.959999) (end 236.22 99.06) (width 0.25) (layer B.Cu) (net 24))
 (segment (start 234.994999 100.285001) (end 235.320001 99.959999) (width 0.25) (layer B.Cu) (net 24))
 (segment (start 232.519999 100.285001) (end 234.994999 100.285001) (width 0.25) (layer B.Cu) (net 24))
 (segment (start 232.310998 100.076) (end 232.519999 100.285001) (width 0.25) (layer B.Cu) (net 24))
 (segment (start 230.632 100.076) (end 232.310998 100.076) (width 0.25) (layer B.Cu) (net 24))
 (segment (start 227.51 139.192) (end 226.06 139.192) (width 0.25) (layer F.Cu) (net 6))
 (segment (start 227.71241 139.192) (end 227.51 139.192) (width 0.25) (layer F.Cu) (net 6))
 (segment (start 230.124 136.78041) (end 227.71241 139.192) (width 0.25) (layer F.Cu) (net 6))
 (segment (start 230.632 94.996) (end 229.606999 96.021001) (width 0.25) (layer F.Cu) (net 6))
 (segment (start 229.606999 96.021001) (end 229.606999 106.689001) (width 0.25) (layer F.Cu) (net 6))
 (segment (start 227.52601 108.76999) (end 227.52601 125.7976) (width 0.25) (layer F.Cu) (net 6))
 (segment (start 227.52601 125.7976) (end 230.124 128.39559) (width 0.25) (layer F.Cu) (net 6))
 (segment (start 229.606999 106.689001) (end 227.52601 108.76999) (width 0.25) (layer F.Cu) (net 6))
 (segment (start 230.124 128.39559) (end 230.124 136.78041) (width 0.25) (layer F.Cu) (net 6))
 (segment (start 214.567999 100.775999) (end 214.567999 102.299999) (width 0.25) (layer F.Cu) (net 4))
 (segment (start 213.868 100.076) (end 214.567999 100.775999) (width 0.25) (layer F.Cu) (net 4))
 (segment (start 214.567999 102.299999) (end 227.076 114.808) (width 0.25) (layer F.Cu) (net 4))
 (segment (start 227.076 114.808) (end 227.076 125.984) (width 0.25) (layer F.Cu) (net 4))
 (segment (start 227.076 125.984) (end 229.616 128.524) (width 0.25) (layer F.Cu) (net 4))
 (segment (start 229.616 128.524) (end 229.616 136.652) (width 0.25) (layer F.Cu) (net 4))
 (segment (start 229.616 136.652) (end 226.06 136.652) (width 0.25) (layer F.Cu) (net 4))
 (segment (start 210.82 97.787208) (end 210.82 99.06) (width 0.25) (layer B.Cu) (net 15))
 (segment (start 212.911209 95.695999) (end 210.82 97.787208) (width 0.25) (layer B.Cu) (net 15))
 (segment (start 213.168001 95.695999) (end 212.911209 95.695999) (width 0.25) (layer B.Cu) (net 15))
 (segment (start 213.868 94.996) (end 213.168001 95.695999) (width 0.25) (layer B.Cu) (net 15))
 (segment (start 219.964 110.744) (end 222.504 110.744) (width 0.25) (layer B.Cu) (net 2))
 (segment (start 213.614001 117.093999) (end 219.964 110.744) (width 0.25) (layer B.Cu) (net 2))
 (segment (start 213.614001 119.754001) (end 213.614001 117.093999) (width 0.25) (layer B.Cu) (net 2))
 (segment (start 220.98 128.27) (end 220.98 127.12) (width 0.25) (layer B.Cu) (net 2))
 (segment (start 232.520999 99.050999) (end 227.593001 99.050999) (width 0.25) (layer B.Cu) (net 2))
 (segment (start 233.68 99.06) (end 232.53 99.06) (width 0.25) (layer B.Cu) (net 2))
 (segment (start 232.53 99.06) (end 232.520999 99.050999) (width 0.25) (layer B.Cu) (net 2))
 (segment (start 222.504 104.14) (end 222.504 110.744) (width 0.25) (layer B.Cu) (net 2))
 (segment (start 227.593001 99.050999) (end 222.504 104.14) (width 0.25) (layer B.Cu) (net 2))
 (segment (start 208.28 99.06) (end 208.28 97.91) (width 0.25) (layer B.Cu) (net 2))
 (segment (start 245.887999 123.434999) (end 243.332 125.990998) (width 0.25) (layer F.Cu) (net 2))
 (segment (start 248.92 124.46) (end 247.894999 123.434999) (width 0.25) (layer F.Cu) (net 2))
 (segment (start 247.894999 123.434999) (end 245.887999 123.434999) (width 0.25) (layer F.Cu) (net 2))
 (segment (start 237.49 137.28) (end 237.49 138.43) (width 0.25) (layer F.Cu) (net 2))
 (segment (start 237.49 134.366) (end 237.49 137.28) (width 0.25) (layer F.Cu) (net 2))
 (segment (start 243.332 128.524) (end 237.49 134.366) (width 0.25) (layer F.Cu) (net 2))
 (segment (start 243.332 125.990998) (end 243.332 128.524) (width 0.25) (layer F.Cu) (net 2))
 (segment (start 247.784 128.524) (end 243.332 128.524) (width 0.25) (layer F.Cu) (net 2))
 (segment (start 256.54 137.28) (end 247.784 128.524) (width 0.25) (layer F.Cu) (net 2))
 (segment (start 256.54 138.43) (end 256.54 137.28) (width 0.25) (layer F.Cu) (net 2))
 (segment (start 231.393999 129.178001) (end 231.393999 119.633999) (width 0.25) (layer B.Cu) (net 2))
 (segment (start 226.46 134.112) (end 231.393999 129.178001) (width 0.25) (layer B.Cu) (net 2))
 (segment (start 226.06 134.112) (end 226.46 134.112) (width 0.25) (layer B.Cu) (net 2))
 (segment (start 231.393999 119.633999) (end 222.504 110.744) (width 0.25) (layer B.Cu) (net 2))
 (segment (start 245.692601 119.633999) (end 231.393999 119.633999) (width 0.25) (layer B.Cu) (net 2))
 (segment (start 248.92 122.861398) (end 245.692601 119.633999) (width 0.25) (layer B.Cu) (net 2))
 (segment (start 248.92 124.46) (end 248.92 122.861398) (width 0.25) (layer B.Cu) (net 2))
 (segment (start 185.42 137.28) (end 185.42 138.43) (width 0.25) (layer B.Cu) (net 2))
 (segment (start 185.549001 137.150999) (end 185.42 137.28) (width 0.25) (layer B.Cu) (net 2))
 (segment (start 202.040999 137.150999) (end 185.549001 137.150999) (width 0.25) (layer B.Cu) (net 2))
 (segment (start 203.32 138.43) (end 202.040999 137.150999) (width 0.25) (layer B.Cu) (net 2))
 (segment (start 204.47 138.43) (end 203.32 138.43) (width 0.25) (layer B.Cu) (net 2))
 (segment (start 193.04 123.31) (end 193.04 124.46) (width 0.25) (layer B.Cu) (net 2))
 (segment (start 197.605002 122.428) (end 193.922 122.428) (width 0.25) (layer B.Cu) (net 2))
 (segment (start 193.922 122.428) (end 193.04 123.31) (width 0.25) (layer B.Cu) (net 2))
 (segment (start 202.040999 126.863997) (end 197.605002 122.428) (width 0.25) (layer B.Cu) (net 2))
 (segment (start 220.98 129.42) (end 220.98 128.27) (width 0.25) (layer B.Cu) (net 2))
 (segment (start 219.900001 135.237001) (end 220.98 134.157002) (width 0.25) (layer B.Cu) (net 2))
 (segment (start 216.979999 135.237001) (end 219.900001 135.237001) (width 0.25) (layer B.Cu) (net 2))
 (segment (start 213.314998 131.572) (end 216.979999 135.237001) (width 0.25) (layer B.Cu) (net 2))
 (segment (start 202.040999 131.572) (end 213.314998 131.572) (width 0.25) (layer B.Cu) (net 2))
 (segment (start 220.98 134.157002) (end 220.98 129.42) (width 0.25) (layer B.Cu) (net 2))
 (segment (start 202.040999 137.150999) (end 202.040999 131.572) (width 0.25) (layer B.Cu) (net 2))
 (segment (start 202.040999 131.572) (end 202.040999 126.863997) (width 0.25) (layer B.Cu) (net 2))
 (segment (start 222.504 98.171642) (end 222.504 110.744) (width 0.25) (layer B.Cu) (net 2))
 (segment (start 222.504 89.288) (end 222.504 98.171642) (width 0.25) (layer B.Cu) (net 2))
 (segment (start 220.98 87.764) (end 222.504 89.288) (width 0.25) (layer B.Cu) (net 2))
 (segment (start 220.98 86.614) (end 220.98 87.764) (width 0.25) (layer B.Cu) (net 2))
 (segment (start 219.576 86.614) (end 220.98 86.614) (width 0.25) (layer B.Cu) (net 2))
 (segment (start 208.28 97.91) (end 219.576 86.614) (width 0.25) (layer B.Cu) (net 2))
 (segment (start 220.98 127.12) (end 213.614001 119.754001) (width 0.25) (layer B.Cu) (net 2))
 (segment (start 218.04 134.112) (end 218.44 134.112) (width 0.25) (layer B.Cu) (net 1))
 (segment (start 212.09 128.162) (end 218.04 134.112) (width 0.25) (layer B.Cu) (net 1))
 (segment (start 212.09 112.268) (end 212.09 128.162) (width 0.25) (layer B.Cu) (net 1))
 (segment (start 231.648001 110.998001) (end 232.918 112.268) (width 0.25) (layer F.Cu) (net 1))
 (segment (start 231.648001 110.489999) (end 231.648001 110.998001) (width 0.25) (layer F.Cu) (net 1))
 (segment (start 232.918 109.22) (end 231.648001 110.489999) (width 0.25) (layer F.Cu) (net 1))
 (segment (start 213.359999 110.489999) (end 212.09 109.22) (width 0.25) (layer F.Cu) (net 1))
 (segment (start 213.359999 110.998001) (end 213.359999 110.489999) (width 0.25) (layer F.Cu) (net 1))
 (segment (start 212.09 112.268) (end 213.359999 110.998001) (width 0.25) (layer F.Cu) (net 1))
 (segment (start 219.264001 90.615999) (end 219.964 89.916) (width 0.25) (layer B.Cu) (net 1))
 (segment (start 219.264001 91.117001) (end 219.264001 90.615999) (width 0.25) (layer B.Cu) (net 1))
 (segment (start 212.09 98.291002) (end 219.264001 91.117001) (width 0.25) (layer B.Cu) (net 1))
 (segment (start 212.09 109.22) (end 212.09 98.291002) (width 0.25) (layer B.Cu) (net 1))
 (segment (start 220.663999 90.615999) (end 219.964 89.916) (width 0.25) (layer F.Cu) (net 1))
 (segment (start 220.989001 90.941001) (end 220.663999 90.615999) (width 0.25) (layer F.Cu) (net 1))
 (segment (start 228.094003 90.941001) (end 220.989001 90.941001) (width 0.25) (layer F.Cu) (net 1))
 (segment (start 231.657001 94.503999) (end 228.094003 90.941001) (width 0.25) (layer F.Cu) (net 1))
 (segment (start 231.657001 101.831003) (end 231.657001 94.503999) (width 0.25) (layer F.Cu) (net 1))
 (segment (start 231.263501 102.224503) (end 231.657001 101.831003) (width 0.25) (layer F.Cu) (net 1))
 (segment (start 231.263501 110.613501) (end 231.263501 102.224503) (width 0.25) (layer F.Cu) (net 1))
 (segment (start 232.918 112.268) (end 231.263501 110.613501) (width 0.25) (layer F.Cu) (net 1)))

